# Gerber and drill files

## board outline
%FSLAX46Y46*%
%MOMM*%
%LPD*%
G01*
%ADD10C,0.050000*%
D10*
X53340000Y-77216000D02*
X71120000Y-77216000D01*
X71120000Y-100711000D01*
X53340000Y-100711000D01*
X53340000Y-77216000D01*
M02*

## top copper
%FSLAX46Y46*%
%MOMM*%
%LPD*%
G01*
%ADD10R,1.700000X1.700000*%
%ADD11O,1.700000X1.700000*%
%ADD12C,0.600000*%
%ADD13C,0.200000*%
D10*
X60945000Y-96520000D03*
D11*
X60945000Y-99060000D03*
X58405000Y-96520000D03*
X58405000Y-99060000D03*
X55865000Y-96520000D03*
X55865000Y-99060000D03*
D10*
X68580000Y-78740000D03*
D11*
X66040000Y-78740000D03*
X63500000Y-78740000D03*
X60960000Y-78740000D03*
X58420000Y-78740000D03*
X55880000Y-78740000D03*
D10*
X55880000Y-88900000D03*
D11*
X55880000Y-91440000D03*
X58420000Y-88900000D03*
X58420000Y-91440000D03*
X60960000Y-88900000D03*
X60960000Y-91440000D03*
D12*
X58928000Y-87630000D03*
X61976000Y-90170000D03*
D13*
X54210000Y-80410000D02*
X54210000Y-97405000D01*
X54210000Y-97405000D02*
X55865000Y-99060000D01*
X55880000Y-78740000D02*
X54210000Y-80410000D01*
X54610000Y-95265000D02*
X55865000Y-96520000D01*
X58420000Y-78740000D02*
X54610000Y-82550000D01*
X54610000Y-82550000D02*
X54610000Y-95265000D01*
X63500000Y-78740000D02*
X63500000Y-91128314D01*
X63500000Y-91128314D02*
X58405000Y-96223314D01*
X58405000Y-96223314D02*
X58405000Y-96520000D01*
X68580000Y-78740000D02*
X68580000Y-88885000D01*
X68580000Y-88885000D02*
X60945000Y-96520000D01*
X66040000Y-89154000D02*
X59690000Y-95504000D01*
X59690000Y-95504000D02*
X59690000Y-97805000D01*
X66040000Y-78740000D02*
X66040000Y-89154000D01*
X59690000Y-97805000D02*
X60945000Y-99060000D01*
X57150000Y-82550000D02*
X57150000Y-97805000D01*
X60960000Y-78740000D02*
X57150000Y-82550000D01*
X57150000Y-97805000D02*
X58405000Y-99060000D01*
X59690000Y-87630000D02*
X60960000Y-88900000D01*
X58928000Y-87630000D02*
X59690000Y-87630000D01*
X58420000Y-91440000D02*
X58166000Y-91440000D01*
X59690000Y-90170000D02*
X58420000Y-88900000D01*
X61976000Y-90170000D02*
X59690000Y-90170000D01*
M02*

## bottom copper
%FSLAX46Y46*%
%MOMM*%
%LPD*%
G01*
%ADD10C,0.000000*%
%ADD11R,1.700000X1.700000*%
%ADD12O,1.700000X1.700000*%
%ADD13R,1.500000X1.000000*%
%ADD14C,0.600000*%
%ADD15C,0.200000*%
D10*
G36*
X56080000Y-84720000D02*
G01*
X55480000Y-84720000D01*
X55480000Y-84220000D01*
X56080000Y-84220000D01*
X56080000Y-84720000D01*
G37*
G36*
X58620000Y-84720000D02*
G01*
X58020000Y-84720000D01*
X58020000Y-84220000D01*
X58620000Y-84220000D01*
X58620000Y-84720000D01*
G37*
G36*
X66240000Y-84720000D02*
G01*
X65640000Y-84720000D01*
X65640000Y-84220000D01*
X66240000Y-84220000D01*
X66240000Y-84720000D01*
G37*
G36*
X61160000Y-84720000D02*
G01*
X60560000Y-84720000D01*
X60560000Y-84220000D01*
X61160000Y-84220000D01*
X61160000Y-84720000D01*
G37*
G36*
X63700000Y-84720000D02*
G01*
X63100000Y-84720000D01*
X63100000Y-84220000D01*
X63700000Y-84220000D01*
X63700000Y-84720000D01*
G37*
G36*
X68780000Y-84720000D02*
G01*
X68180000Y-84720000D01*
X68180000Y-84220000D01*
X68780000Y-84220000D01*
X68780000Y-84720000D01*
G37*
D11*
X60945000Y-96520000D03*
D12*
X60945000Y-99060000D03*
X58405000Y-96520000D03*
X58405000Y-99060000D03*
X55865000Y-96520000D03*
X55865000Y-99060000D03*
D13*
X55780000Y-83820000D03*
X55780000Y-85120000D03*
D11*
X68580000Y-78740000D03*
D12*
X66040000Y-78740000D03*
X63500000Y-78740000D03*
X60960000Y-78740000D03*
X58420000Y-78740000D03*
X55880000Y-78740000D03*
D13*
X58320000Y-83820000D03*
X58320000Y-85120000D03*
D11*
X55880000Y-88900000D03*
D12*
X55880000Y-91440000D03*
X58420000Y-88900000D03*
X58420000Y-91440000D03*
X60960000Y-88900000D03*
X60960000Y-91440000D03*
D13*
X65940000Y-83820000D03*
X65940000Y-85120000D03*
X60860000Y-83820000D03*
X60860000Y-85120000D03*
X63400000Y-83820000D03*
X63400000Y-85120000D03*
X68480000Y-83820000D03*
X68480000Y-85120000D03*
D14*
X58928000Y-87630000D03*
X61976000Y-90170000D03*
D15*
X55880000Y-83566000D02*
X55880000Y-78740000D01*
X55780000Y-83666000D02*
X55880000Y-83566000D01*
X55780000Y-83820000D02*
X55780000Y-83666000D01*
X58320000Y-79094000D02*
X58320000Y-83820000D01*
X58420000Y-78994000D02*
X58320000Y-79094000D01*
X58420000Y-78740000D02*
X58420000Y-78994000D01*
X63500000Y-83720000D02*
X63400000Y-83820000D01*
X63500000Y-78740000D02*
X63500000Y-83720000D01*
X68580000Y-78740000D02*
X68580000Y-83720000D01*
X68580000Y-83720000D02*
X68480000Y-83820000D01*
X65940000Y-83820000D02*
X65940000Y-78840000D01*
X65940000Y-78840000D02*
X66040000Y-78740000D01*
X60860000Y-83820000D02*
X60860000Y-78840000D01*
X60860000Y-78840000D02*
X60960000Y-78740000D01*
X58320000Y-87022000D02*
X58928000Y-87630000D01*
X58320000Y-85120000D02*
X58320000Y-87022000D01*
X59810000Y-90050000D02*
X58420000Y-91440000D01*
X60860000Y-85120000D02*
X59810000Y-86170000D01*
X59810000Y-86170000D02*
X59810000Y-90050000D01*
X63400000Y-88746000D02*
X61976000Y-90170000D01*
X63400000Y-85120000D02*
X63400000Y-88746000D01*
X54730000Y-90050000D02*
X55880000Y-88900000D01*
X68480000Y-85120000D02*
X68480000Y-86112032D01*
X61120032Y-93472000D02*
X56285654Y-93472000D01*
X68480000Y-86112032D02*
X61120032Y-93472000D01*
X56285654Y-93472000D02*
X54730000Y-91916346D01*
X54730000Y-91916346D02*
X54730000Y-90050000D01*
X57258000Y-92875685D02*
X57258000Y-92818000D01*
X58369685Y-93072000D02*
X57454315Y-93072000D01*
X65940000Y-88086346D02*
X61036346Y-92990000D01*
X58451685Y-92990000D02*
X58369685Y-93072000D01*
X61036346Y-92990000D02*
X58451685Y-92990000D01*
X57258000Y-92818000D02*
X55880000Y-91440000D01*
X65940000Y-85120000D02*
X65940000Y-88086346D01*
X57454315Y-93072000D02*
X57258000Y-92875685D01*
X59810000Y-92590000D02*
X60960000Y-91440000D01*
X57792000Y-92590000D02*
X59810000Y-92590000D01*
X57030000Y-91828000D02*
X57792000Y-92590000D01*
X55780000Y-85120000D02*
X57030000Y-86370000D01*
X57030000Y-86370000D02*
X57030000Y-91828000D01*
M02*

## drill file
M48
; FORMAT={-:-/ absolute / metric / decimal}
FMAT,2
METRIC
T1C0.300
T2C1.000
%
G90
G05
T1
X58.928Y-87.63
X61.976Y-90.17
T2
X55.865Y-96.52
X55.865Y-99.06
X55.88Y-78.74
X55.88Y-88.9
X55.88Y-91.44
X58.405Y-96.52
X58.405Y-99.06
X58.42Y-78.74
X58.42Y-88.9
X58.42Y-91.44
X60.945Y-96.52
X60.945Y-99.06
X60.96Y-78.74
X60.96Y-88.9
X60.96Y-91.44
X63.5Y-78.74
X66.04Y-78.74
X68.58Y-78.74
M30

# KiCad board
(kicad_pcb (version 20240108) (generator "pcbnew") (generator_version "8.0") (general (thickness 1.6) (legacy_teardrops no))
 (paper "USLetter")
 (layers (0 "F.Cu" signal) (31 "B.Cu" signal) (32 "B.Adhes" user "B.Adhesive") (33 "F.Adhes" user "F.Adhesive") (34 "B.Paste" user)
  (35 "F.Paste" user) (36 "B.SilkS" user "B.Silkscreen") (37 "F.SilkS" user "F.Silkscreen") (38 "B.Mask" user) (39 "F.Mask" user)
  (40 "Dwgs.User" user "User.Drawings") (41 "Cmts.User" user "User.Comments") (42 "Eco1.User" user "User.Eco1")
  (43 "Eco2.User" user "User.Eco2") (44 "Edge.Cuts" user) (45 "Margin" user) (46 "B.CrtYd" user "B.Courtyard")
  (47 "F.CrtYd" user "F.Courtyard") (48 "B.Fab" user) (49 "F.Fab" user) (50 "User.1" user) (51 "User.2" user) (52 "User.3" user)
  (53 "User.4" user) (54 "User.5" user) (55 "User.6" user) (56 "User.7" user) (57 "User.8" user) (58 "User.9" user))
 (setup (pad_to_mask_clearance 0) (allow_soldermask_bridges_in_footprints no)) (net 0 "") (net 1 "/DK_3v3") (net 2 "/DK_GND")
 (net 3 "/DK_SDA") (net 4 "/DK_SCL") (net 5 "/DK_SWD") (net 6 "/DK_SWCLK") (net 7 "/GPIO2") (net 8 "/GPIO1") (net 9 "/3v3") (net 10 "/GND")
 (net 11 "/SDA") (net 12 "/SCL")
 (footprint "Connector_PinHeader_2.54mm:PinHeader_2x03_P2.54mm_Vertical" (layer "F.Cu") (at 60.945 96.52 -90)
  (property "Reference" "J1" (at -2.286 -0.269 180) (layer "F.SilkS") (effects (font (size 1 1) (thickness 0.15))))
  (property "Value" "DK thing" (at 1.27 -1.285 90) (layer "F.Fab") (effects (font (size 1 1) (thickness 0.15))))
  (pad "1" thru_hole rect (at 0 0 270) (size 1.7 1.7) (drill 1) (layers "*.Cu" "*.Mask") (remove_unused_layers no) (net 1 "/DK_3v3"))
  (pad "2" thru_hole oval (at 2.54 0 270) (size 1.7 1.7) (drill 1) (layers "*.Cu" "*.Mask") (remove_unused_layers no) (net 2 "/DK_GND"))
  (pad "3" thru_hole oval (at 0 2.54 270) (size 1.7 1.7) (drill 1) (layers "*.Cu" "*.Mask") (remove_unused_layers no) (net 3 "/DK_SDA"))
  (pad "4" thru_hole oval (at 2.54 2.54 270) (size 1.7 1.7) (drill 1) (layers "*.Cu" "*.Mask") (remove_unused_layers no) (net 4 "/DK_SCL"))
  (pad "5" thru_hole oval (at 0 5.08 270) (size 1.7 1.7) (drill 1) (layers "*.Cu" "*.Mask") (remove_unused_layers no) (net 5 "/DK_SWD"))
  (pad "6" thru_hole oval (at 2.54 5.08 270) (size 1.7 1.7) (drill 1) (layers "*.Cu" "*.Mask") (remove_unused_layers no) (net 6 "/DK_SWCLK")))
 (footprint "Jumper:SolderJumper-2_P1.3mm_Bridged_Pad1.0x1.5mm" (layer "B.Cu") (at 55.78 84.47 -90)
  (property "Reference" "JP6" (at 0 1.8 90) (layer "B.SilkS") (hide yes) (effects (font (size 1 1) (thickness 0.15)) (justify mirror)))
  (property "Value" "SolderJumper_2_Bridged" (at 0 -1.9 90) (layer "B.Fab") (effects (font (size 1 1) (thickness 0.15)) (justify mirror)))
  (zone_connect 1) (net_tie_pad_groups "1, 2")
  (fp_poly (pts (xy -0.25 0.3) (xy 0.25 0.3) (xy 0.25 -0.3) (xy -0.25 -0.3)) (stroke (width 0) (type solid)) (fill solid) (layer "B.Cu"))
  (pad "1" smd rect (at -0.65 0 270) (size 1 1.5) (layers "B.Cu" "B.Mask") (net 6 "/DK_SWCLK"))
  (pad "2" smd rect (at 0.65 0 270) (size 1 1.5) (layers "B.Cu" "B.Mask") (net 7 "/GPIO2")))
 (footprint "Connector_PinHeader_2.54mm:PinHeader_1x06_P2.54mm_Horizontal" (layer "B.Cu") (at 68.58 78.74 90)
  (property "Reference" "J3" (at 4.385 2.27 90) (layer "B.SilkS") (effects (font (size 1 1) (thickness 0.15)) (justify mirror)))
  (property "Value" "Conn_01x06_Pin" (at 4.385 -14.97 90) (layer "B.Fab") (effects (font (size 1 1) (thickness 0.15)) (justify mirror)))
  (pad "1" thru_hole rect (at 0 0 90) (size 1.7 1.7) (drill 1) (layers "*.Cu" "*.Mask") (remove_unused_layers no) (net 1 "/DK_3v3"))
  (pad "2" thru_hole oval (at 0 -2.54 90) (size 1.7 1.7) (drill 1) (layers "*.Cu" "*.Mask") (remove_unused_layers no) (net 2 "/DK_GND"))
  (pad "3" thru_hole oval (at 0 -5.08 90) (size 1.7 1.7) (drill 1) (layers "*.Cu" "*.Mask") (remove_unused_layers no) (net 3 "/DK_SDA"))
  (pad "4" thru_hole oval (at 0 -7.62 90) (size 1.7 1.7) (drill 1) (layers "*.Cu" "*.Mask") (remove_unused_layers no) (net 4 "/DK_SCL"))
  (pad "5" thru_hole oval (at 0 -10.16 90) (size 1.7 1.7) (drill 1) (layers "*.Cu" "*.Mask") (remove_unused_layers no) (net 5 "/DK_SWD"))
  (pad "6" thru_hole oval (at 0 -12.7 90) (size 1.7 1.7) (drill 1) (layers "*.Cu" "*.Mask") (remove_unused_layers no) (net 6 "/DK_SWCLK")))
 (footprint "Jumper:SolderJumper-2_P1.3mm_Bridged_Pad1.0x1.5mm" (layer "B.Cu") (at 58.32 84.47 -90)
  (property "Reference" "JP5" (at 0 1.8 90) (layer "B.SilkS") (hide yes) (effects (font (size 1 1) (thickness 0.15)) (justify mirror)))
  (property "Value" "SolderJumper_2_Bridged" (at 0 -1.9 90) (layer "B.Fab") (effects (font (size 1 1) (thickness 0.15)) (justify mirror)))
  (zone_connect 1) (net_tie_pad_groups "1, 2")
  (fp_poly (pts (xy -0.25 0.3) (xy 0.25 0.3) (xy 0.25 -0.3) (xy -0.25 -0.3)) (stroke (width 0) (type solid)) (fill solid) (layer "B.Cu"))
  (pad "1" smd rect (at -0.65 0 270) (size 1 1.5) (layers "B.Cu" "B.Mask") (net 5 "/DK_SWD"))
  (pad "2" smd rect (at 0.65 0 270) (size 1 1.5) (layers "B.Cu" "B.Mask") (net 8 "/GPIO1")))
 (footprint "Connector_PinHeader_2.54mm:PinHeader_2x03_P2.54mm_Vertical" (layer "B.Cu") (at 55.88 88.9 -90)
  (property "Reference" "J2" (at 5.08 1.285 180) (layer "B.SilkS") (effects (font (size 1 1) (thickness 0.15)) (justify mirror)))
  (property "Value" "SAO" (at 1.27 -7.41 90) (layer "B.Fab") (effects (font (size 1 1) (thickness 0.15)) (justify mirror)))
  (pad "1" thru_hole rect (at 0 0 270) (size 1.7 1.7) (drill 1) (layers "*.Cu" "*.Mask") (remove_unused_layers no) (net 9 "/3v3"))
  (pad "2" thru_hole oval (at 2.54 0 270) (size 1.7 1.7) (drill 1) (layers "*.Cu" "*.Mask") (remove_unused_layers no) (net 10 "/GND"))
  (pad "3" thru_hole oval (at 0 -2.54 270) (size 1.7 1.7) (drill 1) (layers "*.Cu" "*.Mask") (remove_unused_layers no) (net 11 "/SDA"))
  (pad "4" thru_hole oval (at 2.54 -2.54 270) (size 1.7 1.7) (drill 1) (layers "*.Cu" "*.Mask") (remove_unused_layers no) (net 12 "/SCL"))
  (pad "5" thru_hole oval (at 0 -5.08 270) (size 1.7 1.7) (drill 1) (layers "*.Cu" "*.Mask") (remove_unused_layers no) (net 8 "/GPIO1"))
  (pad "6" thru_hole oval (at 2.54 -5.08 270) (size 1.7 1.7) (drill 1) (layers "*.Cu" "*.Mask") (remove_unused_layers no) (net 7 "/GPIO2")))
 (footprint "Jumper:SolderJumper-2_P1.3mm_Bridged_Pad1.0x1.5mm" (layer "B.Cu") (at 65.94 84.47 -90)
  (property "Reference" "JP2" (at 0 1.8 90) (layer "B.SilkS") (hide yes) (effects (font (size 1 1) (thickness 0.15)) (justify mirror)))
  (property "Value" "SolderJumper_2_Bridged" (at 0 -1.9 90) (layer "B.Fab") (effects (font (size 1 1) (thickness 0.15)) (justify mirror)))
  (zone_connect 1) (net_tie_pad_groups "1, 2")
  (fp_poly (pts (xy -0.25 0.3) (xy 0.25 0.3) (xy 0.25 -0.3) (xy -0.25 -0.3)) (stroke (width 0) (type solid)) (fill solid) (layer "B.Cu"))
  (pad "1" smd rect (at -0.65 0 270) (size 1 1.5) (layers "B.Cu" "B.Mask") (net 2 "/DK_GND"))
  (pad "2" smd rect (at 0.65 0 270) (size 1 1.5) (layers "B.Cu" "B.Mask") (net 10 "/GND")))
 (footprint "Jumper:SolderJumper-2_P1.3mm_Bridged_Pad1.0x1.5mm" (layer "B.Cu") (at 60.86 84.47 -90)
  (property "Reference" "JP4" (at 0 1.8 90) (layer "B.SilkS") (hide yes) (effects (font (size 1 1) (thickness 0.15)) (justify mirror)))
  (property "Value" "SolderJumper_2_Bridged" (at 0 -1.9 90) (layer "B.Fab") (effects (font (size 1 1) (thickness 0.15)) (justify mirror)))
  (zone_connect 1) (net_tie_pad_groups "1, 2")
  (fp_poly (pts (xy -0.25 0.3) (xy 0.25 0.3) (xy 0.25 -0.3) (xy -0.25 -0.3)) (stroke (width 0) (type solid)) (fill solid) (layer "B.Cu"))
  (pad "1" smd rect (at -0.65 0 270) (size 1 1.5) (layers "B.Cu" "B.Mask") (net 4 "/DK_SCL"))
  (pad "2" smd rect (at 0.65 0 270) (size 1 1.5) (layers "B.Cu" "B.Mask") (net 12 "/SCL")))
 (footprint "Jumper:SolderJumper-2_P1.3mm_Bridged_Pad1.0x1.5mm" (layer "B.Cu") (at 63.4 84.47 -90)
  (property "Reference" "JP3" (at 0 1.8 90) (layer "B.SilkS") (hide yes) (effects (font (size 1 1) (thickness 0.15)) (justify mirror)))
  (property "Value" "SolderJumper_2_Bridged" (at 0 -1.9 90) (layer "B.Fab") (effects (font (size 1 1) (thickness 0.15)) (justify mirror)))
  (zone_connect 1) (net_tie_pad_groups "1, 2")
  (fp_poly (pts (xy -0.25 0.3) (xy 0.25 0.3) (xy 0.25 -0.3) (xy -0.25 -0.3)) (stroke (width 0) (type solid)) (fill solid) (layer "B.Cu"))
  (pad "1" smd rect (at -0.65 0 270) (size 1 1.5) (layers "B.Cu" "B.Mask") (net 3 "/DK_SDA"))
  (pad "2" smd rect (at 0.65 0 270) (size 1 1.5) (layers "B.Cu" "B.Mask") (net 11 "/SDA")))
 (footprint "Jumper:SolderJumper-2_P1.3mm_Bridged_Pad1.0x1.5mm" (layer "B.Cu") (at 68.48 84.47 -90)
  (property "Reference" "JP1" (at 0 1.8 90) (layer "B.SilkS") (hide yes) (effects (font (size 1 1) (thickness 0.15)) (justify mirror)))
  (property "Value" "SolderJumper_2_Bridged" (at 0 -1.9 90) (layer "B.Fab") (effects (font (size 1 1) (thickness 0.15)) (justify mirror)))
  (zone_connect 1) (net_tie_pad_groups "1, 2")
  (fp_poly (pts (xy -0.25 0.3) (xy 0.25 0.3) (xy 0.25 -0.3) (xy -0.25 -0.3)) (stroke (width 0) (type solid)) (fill solid) (layer "B.Cu"))
  (pad "1" smd rect (at -0.65 0 270) (size 1 1.5) (layers "B.Cu" "B.Mask") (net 1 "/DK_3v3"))
  (pad "2" smd rect (at 0.65 0 270) (size 1 1.5) (layers "B.Cu" "B.Mask") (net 9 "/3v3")))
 (gr_rect (start 53.34 77.216) (end 71.12 100.711) (stroke (width 0.05) (type default)) (fill none) (layer "Edge.Cuts"))
 (segment (start 54.21 80.41) (end 54.21 97.405) (width 0.2) (layer "F.Cu") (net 6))
 (segment (start 54.21 97.405) (end 55.865 99.06) (width 0.2) (layer "F.Cu") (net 6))
 (segment (start 55.88 78.74) (end 54.21 80.41) (width 0.2) (layer "F.Cu") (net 6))
 (segment (start 55.88 83.566) (end 55.88 78.74) (width 0.2) (layer "B.Cu") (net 6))
 (segment (start 55.78 83.666) (end 55.88 83.566) (width 0.2) (layer "B.Cu") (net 6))
 (segment (start 55.78 83.82) (end 55.78 83.666) (width 0.2) (layer "B.Cu") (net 6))
 (segment (start 54.61 95.265) (end 55.865 96.52) (width 0.2) (layer "F.Cu") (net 5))
 (segment (start 58.42 78.74) (end 54.61 82.55) (width 0.2) (layer "F.Cu") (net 5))
 (segment (start 54.61 82.55) (end 54.61 95.265) (width 0.2) (layer "F.Cu") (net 5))
 (segment (start 58.32 79.094) (end 58.32 83.82) (width 0.2) (layer "B.Cu") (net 5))
 (segment (start 58.42 78.994) (end 58.32 79.094) (width 0.2) (layer "B.Cu") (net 5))
 (segment (start 58.42 78.74) (end 58.42 78.994) (width 0.2) (layer "B.Cu") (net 5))
 (segment (start 63.5 78.74) (end 63.5 91.128314) (width 0.2) (layer "F.Cu") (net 3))
 (segment (start 63.5 91.128314) (end 58.405 96.223314) (width 0.2) (layer "F.Cu") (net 3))
 (segment (start 58.405 96.223314) (end 58.405 96.52) (width 0.2) (layer "F.Cu") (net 3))
 (segment (start 63.5 83.72) (end 63.4 83.82) (width 0.2) (layer "B.Cu") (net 3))
 (segment (start 63.5 78.74) (end 63.5 83.72) (width 0.2) (layer "B.Cu") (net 3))
 (segment (start 68.58 78.74) (end 68.58 88.885) (width 0.2) (layer "F.Cu") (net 1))
 (segment (start 68.58 88.885) (end 60.945 96.52) (width 0.2) (layer "F.Cu") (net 1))
 (segment (start 68.58 78.74) (end 68.58 83.72) (width 0.2) (layer "B.Cu") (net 1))
 (segment (start 68.58 83.72) (end 68.48 83.82) (width 0.2) (layer "B.Cu") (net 1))
 (segment (start 66.04 89.154) (end 59.69 95.504) (width 0.2) (layer "F.Cu") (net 2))
 (segment (start 59.69 95.504) (end 59.69 97.805) (width 0.2) (layer "F.Cu") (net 2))
 (segment (start 66.04 78.74) (end 66.04 89.154) (width 0.2) (layer "F.Cu") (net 2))
 (segment (start 59.69 97.805) (end 60.945 99.06) (width 0.2) (layer "F.Cu") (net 2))
 (segment (start 65.94 83.82) (end 65.94 78.84) (width 0.2) (layer "B.Cu") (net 2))
 (segment (start 65.94 78.84) (end 66.04 78.74) (width 0.2) (layer "B.Cu") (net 2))
 (segment (start 57.15 82.55) (end 57.15 97.805) (width 0.2) (layer "F.Cu") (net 4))
 (segment (start 60.96 78.74) (end 57.15 82.55) (width 0.2) (layer "F.Cu") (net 4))
 (segment (start 57.15 97.805) (end 58.405 99.06) (width 0.2) (layer "F.Cu") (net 4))
 (segment (start 60.86 83.82) (end 60.86 78.84) (width 0.2) (layer "B.Cu") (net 4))
 (segment (start 60.86 78.84) (end 60.96 78.74) (width 0.2) (layer "B.Cu") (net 4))
 (segment (start 59.69 87.63) (end 60.96 88.9) (width 0.2) (layer "F.Cu") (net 8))
 (segment (start 58.928 87.63) (end 59.69 87.63) (width 0.2) (layer "F.Cu") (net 8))
 (via (at 58.928 87.63) (size 0.6) (drill 0.3) (layers "F.Cu" "B.Cu") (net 8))
 (segment (start 58.32 87.022) (end 58.928 87.63) (width 0.2) (layer "B.Cu") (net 8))
 (segment (start 58.32 85.12) (end 58.32 87.022) (width 0.2) (layer "B.Cu") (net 8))
 (segment (start 58.42 91.44) (end 58.166 91.44) (width 0.2) (layer "F.Cu") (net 12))
 (segment (start 59.81 90.05) (end 58.42 91.44) (width 0.2) (layer "B.Cu") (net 12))
 (segment (start 60.86 85.12) (end 59.81 86.17) (width 0.2) (layer "B.Cu") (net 12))
 (segment (start 59.81 86.17) (end 59.81 90.05) (width 0.2) (layer "B.Cu") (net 12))
 (segment (start 59.69 90.17) (end 58.42 88.9) (width 0.2) (layer "F.Cu") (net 11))
 (segment (start 61.976 90.17) (end 59.69 90.17) (width 0.2) (layer "F.Cu") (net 11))
 (via (at 61.976 90.17) (size 0.6) (drill 0.3) (layers "F.Cu" "B.Cu") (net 11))
 (segment (start 63.4 88.746) (end 61.976 90.17) (width 0.2) (layer "B.Cu") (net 11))
 (segment (start 63.4 85.12) (end 63.4 88.746) (width 0.2) (layer "B.Cu") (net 11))
 (segment (start 54.73 90.05) (end 55.88 88.9) (width 0.2) (layer "B.Cu") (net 9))
 (segment (start 68.48 85.12) (end 68.48 86.112032) (width 0.2) (layer "B.Cu") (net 9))
 (segment (start 61.120032 93.472) (end 56.285654 93.472) (width 0.2) (layer "B.Cu") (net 9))
 (segment (start 68.48 86.112032) (end 61.120032 93.472) (width 0.2) (layer "B.Cu") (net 9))
 (segment (start 56.285654 93.472) (end 54.73 91.916346) (width 0.2) (layer "B.Cu") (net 9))
 (segment (start 54.73 91.916346) (end 54.73 90.05) (width 0.2) (layer "B.Cu") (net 9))
 (segment (start 57.258 92.875685) (end 57.258 92.818) (width 0.2) (layer "B.Cu") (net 10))
 (segment (start 58.369685 93.072) (end 57.454315 93.072) (width 0.2) (layer "B.Cu") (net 10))
 (segment (start 65.94 88.086346) (end 61.036346 92.99) (width 0.2) (layer "B.Cu") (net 10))
 (segment (start 58.451685 92.99) (end 58.369685 93.072) (width 0.2) (layer "B.Cu") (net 10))
 (segment (start 61.036346 92.99) (end 58.451685 92.99) (width 0.2) (layer "B.Cu") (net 10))
 (segment (start 57.258 92.818) (end 55.88 91.44) (width 0.2) (layer "B.Cu") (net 10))
 (segment (start 65.94 85.12) (end 65.94 88.086346) (width 0.2) (layer "B.Cu") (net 10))
 (segment (start 57.454315 93.072) (end 57.258 92.875685) (width 0.2) (layer "B.Cu") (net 10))
 (segment (start 59.81 92.59) (end 60.96 91.44) (width 0.2) (layer "B.Cu") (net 7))
 (segment (start 57.792 92.59) (end 59.81 92.59) (width 0.2) (layer "B.Cu") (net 7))
 (segment (start 57.03 91.828) (end 57.792 92.59) (width 0.2) (layer "B.Cu") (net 7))
 (segment (start 55.78 85.12) (end 57.03 86.37) (width 0.2) (layer "B.Cu") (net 7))
 (segment (start 57.03 86.37) (end 57.03 91.828) (width 0.2) (layer "B.Cu") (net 7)))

